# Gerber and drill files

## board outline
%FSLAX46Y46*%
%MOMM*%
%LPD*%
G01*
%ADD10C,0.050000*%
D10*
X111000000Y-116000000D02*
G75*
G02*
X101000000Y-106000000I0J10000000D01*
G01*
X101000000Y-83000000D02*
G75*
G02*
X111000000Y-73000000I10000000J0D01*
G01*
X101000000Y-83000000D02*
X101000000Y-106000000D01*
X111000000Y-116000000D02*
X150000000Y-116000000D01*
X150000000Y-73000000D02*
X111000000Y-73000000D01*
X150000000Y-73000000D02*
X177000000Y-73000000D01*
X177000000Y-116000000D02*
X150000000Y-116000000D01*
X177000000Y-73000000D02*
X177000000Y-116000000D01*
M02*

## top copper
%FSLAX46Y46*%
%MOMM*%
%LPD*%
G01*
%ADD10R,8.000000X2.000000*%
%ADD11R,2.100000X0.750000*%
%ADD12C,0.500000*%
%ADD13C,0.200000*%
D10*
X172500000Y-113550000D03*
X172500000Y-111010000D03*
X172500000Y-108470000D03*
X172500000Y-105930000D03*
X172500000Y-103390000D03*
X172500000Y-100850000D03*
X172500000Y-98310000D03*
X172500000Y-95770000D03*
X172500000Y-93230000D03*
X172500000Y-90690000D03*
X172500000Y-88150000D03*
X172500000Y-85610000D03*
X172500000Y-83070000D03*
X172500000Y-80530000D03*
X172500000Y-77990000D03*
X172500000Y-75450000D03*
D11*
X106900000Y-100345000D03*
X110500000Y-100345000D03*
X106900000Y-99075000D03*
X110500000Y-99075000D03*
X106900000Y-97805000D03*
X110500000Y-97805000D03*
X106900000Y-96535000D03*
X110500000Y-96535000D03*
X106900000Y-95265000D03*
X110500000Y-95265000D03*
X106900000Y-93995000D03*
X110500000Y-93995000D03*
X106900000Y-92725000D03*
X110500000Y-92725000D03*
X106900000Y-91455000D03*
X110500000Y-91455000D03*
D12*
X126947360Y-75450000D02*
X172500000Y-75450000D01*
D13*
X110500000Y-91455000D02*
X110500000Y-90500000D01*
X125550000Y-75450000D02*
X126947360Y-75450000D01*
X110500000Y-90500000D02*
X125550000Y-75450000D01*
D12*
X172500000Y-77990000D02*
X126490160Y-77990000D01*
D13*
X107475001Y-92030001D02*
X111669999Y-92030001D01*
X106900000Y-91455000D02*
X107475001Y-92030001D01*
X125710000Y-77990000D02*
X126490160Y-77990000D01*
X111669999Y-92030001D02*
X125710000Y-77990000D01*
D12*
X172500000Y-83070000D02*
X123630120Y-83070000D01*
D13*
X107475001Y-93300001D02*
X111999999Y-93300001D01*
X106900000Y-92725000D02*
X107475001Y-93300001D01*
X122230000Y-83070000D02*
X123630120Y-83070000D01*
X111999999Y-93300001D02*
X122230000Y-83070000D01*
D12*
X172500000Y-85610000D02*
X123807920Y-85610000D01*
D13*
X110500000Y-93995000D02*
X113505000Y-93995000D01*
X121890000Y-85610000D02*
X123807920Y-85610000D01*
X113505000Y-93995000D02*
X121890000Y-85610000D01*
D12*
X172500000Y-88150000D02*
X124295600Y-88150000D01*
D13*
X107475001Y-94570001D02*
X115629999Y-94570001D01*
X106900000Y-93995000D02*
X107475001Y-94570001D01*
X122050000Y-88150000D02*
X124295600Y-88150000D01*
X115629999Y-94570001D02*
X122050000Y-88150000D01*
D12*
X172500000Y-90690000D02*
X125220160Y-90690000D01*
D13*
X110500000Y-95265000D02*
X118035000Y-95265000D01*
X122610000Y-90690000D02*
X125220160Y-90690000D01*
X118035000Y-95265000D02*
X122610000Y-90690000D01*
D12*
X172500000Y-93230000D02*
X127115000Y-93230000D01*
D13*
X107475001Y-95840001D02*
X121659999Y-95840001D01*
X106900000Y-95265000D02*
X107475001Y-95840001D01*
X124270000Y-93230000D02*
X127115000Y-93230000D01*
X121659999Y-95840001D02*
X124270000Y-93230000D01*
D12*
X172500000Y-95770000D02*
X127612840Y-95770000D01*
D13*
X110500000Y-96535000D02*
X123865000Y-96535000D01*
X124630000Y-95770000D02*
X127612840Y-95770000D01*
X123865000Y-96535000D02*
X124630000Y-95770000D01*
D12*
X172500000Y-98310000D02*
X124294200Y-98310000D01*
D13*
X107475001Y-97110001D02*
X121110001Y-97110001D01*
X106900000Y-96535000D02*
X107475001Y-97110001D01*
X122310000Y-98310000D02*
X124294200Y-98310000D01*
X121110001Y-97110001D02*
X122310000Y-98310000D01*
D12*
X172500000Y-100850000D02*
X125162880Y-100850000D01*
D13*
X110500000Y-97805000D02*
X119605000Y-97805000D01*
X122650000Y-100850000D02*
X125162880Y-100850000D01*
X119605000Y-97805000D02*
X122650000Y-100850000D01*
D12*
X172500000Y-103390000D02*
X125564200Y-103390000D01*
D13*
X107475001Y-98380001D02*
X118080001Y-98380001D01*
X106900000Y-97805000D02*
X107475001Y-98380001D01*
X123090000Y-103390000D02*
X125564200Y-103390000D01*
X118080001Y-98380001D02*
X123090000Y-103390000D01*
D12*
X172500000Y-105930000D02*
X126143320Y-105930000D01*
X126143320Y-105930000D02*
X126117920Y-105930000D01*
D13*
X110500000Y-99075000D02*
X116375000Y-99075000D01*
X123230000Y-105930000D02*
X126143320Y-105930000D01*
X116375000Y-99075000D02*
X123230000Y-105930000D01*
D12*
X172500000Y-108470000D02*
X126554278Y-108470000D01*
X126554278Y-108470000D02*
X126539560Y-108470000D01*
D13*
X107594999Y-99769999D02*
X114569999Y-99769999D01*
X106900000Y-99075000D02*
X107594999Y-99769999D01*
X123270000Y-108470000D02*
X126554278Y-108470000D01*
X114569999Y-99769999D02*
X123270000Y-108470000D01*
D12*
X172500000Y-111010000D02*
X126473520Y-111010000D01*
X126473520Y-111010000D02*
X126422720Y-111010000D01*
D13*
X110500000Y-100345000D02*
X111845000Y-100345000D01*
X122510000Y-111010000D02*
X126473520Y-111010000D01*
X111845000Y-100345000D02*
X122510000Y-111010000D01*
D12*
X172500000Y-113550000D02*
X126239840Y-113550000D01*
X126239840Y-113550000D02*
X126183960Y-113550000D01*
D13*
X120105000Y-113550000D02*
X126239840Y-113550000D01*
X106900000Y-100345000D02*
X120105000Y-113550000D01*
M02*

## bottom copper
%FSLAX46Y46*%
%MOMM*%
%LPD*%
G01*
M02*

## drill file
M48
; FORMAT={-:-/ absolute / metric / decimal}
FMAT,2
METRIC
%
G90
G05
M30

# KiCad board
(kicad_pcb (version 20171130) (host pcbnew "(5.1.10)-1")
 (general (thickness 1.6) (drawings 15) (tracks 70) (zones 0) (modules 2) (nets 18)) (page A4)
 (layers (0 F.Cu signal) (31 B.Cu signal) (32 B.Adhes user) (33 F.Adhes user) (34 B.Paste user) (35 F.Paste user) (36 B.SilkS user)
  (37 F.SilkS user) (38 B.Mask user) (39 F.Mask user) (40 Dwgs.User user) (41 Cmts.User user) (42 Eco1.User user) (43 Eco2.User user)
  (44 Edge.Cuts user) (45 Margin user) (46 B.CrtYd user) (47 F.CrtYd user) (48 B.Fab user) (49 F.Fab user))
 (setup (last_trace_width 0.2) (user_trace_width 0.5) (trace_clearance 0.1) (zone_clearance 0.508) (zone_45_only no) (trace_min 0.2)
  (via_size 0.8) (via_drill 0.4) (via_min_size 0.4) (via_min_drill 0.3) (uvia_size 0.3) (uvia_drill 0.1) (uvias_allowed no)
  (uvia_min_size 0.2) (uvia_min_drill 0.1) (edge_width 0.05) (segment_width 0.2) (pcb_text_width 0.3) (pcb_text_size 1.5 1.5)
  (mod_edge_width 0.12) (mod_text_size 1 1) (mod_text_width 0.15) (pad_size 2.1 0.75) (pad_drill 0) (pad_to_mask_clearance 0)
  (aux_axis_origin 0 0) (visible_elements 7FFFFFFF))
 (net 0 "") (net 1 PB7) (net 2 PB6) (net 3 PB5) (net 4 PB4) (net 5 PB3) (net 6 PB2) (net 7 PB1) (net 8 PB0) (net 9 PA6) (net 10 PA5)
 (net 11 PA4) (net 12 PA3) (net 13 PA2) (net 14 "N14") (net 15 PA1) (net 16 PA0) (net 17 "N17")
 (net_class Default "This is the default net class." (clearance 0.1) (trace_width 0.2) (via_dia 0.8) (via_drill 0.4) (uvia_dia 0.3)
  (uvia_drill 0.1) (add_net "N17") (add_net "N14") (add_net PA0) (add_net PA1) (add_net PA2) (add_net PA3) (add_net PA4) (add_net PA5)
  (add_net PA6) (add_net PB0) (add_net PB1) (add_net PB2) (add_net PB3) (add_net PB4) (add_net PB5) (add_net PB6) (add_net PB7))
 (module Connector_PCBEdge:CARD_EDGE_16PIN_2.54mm (layer F.Cu) (at 172.5 94.5 90)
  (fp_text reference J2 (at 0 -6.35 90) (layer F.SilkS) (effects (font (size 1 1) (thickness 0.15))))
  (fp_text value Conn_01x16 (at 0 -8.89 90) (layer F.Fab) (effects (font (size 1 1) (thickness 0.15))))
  (pad 16 connect rect (at -19.05 0 90) (size 2 8) (layers F.Cu F.Mask) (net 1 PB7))
  (pad 15 connect rect (at -16.51 0 90) (size 2 8) (layers F.Cu F.Mask) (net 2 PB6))
  (pad 14 connect rect (at -13.97 0 90) (size 2 8) (layers F.Cu F.Mask) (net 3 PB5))
  (pad 13 connect rect (at -11.43 0 90) (size 2 8) (layers F.Cu F.Mask) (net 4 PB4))
  (pad 12 connect rect (at -8.89 0 90) (size 2 8) (layers F.Cu F.Mask) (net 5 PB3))
  (pad 11 connect rect (at -6.35 0 90) (size 2 8) (layers F.Cu F.Mask) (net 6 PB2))
  (pad 10 connect rect (at -3.81 0 90) (size 2 8) (layers F.Cu F.Mask) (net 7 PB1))
  (pad 9 connect rect (at -1.27 0 90) (size 2 8) (layers F.Cu F.Mask) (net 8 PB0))
  (pad 8 connect rect (at 1.27 0 90) (size 2 8) (layers F.Cu F.Mask) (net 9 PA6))
  (pad 7 connect rect (at 3.81 0 90) (size 2 8) (layers F.Cu F.Mask) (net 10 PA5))
  (pad 6 connect rect (at 6.35 0 90) (size 2 8) (layers F.Cu F.Mask) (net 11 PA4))
  (pad 5 connect rect (at 8.89 0 90) (size 2 8) (layers F.Cu F.Mask) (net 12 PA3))
  (pad 4 connect rect (at 11.43 0 90) (size 2 8) (layers F.Cu F.Mask) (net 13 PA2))
  (pad 3 connect rect (at 13.97 0 90) (size 2 8) (layers F.Cu F.Mask) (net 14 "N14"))
  (pad 2 connect rect (at 16.51 0 90) (size 2 8) (layers F.Cu F.Mask) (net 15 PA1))
  (pad 1 connect rect (at 19.05 0 90) (size 2 8) (layers F.Cu F.Mask) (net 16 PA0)))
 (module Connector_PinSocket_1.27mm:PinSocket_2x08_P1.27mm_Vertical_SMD (layer F.Cu) (at 108.7 95.9)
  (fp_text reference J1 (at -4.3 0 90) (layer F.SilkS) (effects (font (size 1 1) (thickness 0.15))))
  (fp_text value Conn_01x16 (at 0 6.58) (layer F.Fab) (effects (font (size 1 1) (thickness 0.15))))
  (pad 16 smd rect (at -1.8 4.445) (size 2.1 0.75) (layers F.Cu F.Paste F.Mask) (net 1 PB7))
  (pad 15 smd rect (at 1.8 4.445) (size 2.1 0.75) (layers F.Cu F.Paste F.Mask) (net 2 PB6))
  (pad 14 smd rect (at -1.8 3.175) (size 2.1 0.75) (layers F.Cu F.Paste F.Mask) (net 3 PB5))
  (pad 13 smd rect (at 1.8 3.175) (size 2.1 0.75) (layers F.Cu F.Paste F.Mask) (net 4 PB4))
  (pad 12 smd rect (at -1.8 1.905) (size 2.1 0.75) (layers F.Cu F.Paste F.Mask) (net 5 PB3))
  (pad 11 smd rect (at 1.8 1.905) (size 2.1 0.75) (layers F.Cu F.Paste F.Mask) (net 6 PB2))
  (pad 10 smd rect (at -1.8 0.635) (size 2.1 0.75) (layers F.Cu F.Paste F.Mask) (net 7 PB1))
  (pad 9 smd rect (at 1.8 0.635) (size 2.1 0.75) (layers F.Cu F.Paste F.Mask) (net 8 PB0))
  (pad 8 smd rect (at -1.8 -0.635) (size 2.1 0.75) (layers F.Cu F.Paste F.Mask) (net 9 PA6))
  (pad 7 smd rect (at 1.8 -0.635) (size 2.1 0.75) (layers F.Cu F.Paste F.Mask) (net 10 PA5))
  (pad 6 smd rect (at -1.8 -1.905) (size 2.1 0.75) (layers F.Cu F.Paste F.Mask) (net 11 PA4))
  (pad 5 smd rect (at 1.8 -1.905) (size 2.1 0.75) (layers F.Cu F.Paste F.Mask) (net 12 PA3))
  (pad 4 smd rect (at -1.8 -3.175) (size 2.1 0.75) (layers F.Cu F.Paste F.Mask) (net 13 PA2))
  (pad 3 smd rect (at 1.8 -3.175) (size 2.1 0.75) (layers F.Cu F.Paste F.Mask) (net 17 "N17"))
  (pad 2 smd rect (at -1.8 -4.445) (size 2.1 0.75) (layers F.Cu F.Paste F.Mask) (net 15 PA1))
  (pad 1 smd rect (at 1.8 -4.445) (size 2.1 0.75) (layers F.Cu F.Paste F.Mask) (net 16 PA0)))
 (gr_arc (start 111 106) (end 101 106) (angle -90) (layer Edge.Cuts) (width 0.05))
 (gr_arc (start 111 83) (end 111 73) (angle -90) (layer Edge.Cuts) (width 0.05))
 (gr_line (start 101 83) (end 101 106) (layer Edge.Cuts) (width 0.05))
 (gr_line (start 111 116) (end 150 116) (layer Edge.Cuts) (width 0.05))
 (gr_line (start 150 73) (end 111 73) (layer Edge.Cuts) (width 0.05))
 (gr_line (start 150 73) (end 177 73) (layer Edge.Cuts) (width 0.05))
 (gr_line (start 177 116) (end 150 116) (layer Edge.Cuts) (width 0.05))
 (gr_line (start 177 73) (end 177 116) (layer Edge.Cuts) (width 0.05))
 (segment (start 126.94736 75.45) (end 172.5 75.45) (width 0.5) (layer F.Cu) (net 16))
 (segment (start 110.5 91.455) (end 110.5 90.5) (width 0.2) (layer F.Cu) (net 16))
 (segment (start 125.55 75.45) (end 126.94736 75.45) (width 0.2) (layer F.Cu) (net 16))
 (segment (start 110.5 90.5) (end 125.55 75.45) (width 0.2) (layer F.Cu) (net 16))
 (segment (start 172.5 77.99) (end 126.49016 77.99) (width 0.5) (layer F.Cu) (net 15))
 (segment (start 107.475001 92.030001) (end 111.669999 92.030001) (width 0.2) (layer F.Cu) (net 15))
 (segment (start 106.9 91.455) (end 107.475001 92.030001) (width 0.2) (layer F.Cu) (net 15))
 (segment (start 125.71 77.99) (end 126.49016 77.99) (width 0.2) (layer F.Cu) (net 15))
 (segment (start 111.669999 92.030001) (end 125.71 77.99) (width 0.2) (layer F.Cu) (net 15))
 (segment (start 172.5 83.07) (end 123.63012 83.07) (width 0.5) (layer F.Cu) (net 13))
 (segment (start 107.475001 93.300001) (end 111.999999 93.300001) (width 0.2) (layer F.Cu) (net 13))
 (segment (start 106.9 92.725) (end 107.475001 93.300001) (width 0.2) (layer F.Cu) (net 13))
 (segment (start 122.23 83.07) (end 123.63012 83.07) (width 0.2) (layer F.Cu) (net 13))
 (segment (start 111.999999 93.300001) (end 122.23 83.07) (width 0.2) (layer F.Cu) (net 13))
 (segment (start 172.5 85.61) (end 123.80792 85.61) (width 0.5) (layer F.Cu) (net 12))
 (segment (start 110.5 93.995) (end 113.505 93.995) (width 0.2) (layer F.Cu) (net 12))
 (segment (start 121.89 85.61) (end 123.80792 85.61) (width 0.2) (layer F.Cu) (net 12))
 (segment (start 113.505 93.995) (end 121.89 85.61) (width 0.2) (layer F.Cu) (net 12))
 (segment (start 172.5 88.15) (end 124.2956 88.15) (width 0.5) (layer F.Cu) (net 11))
 (segment (start 107.475001 94.570001) (end 115.629999 94.570001) (width 0.2) (layer F.Cu) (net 11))
 (segment (start 106.9 93.995) (end 107.475001 94.570001) (width 0.2) (layer F.Cu) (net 11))
 (segment (start 122.05 88.15) (end 124.2956 88.15) (width 0.2) (layer F.Cu) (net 11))
 (segment (start 115.629999 94.570001) (end 122.05 88.15) (width 0.2) (layer F.Cu) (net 11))
 (segment (start 172.5 90.69) (end 125.22016 90.69) (width 0.5) (layer F.Cu) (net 10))
 (segment (start 110.5 95.265) (end 118.035 95.265) (width 0.2) (layer F.Cu) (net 10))
 (segment (start 122.61 90.69) (end 125.22016 90.69) (width 0.2) (layer F.Cu) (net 10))
 (segment (start 118.035 95.265) (end 122.61 90.69) (width 0.2) (layer F.Cu) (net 10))
 (segment (start 172.5 93.23) (end 127.115 93.23) (width 0.5) (layer F.Cu) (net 9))
 (segment (start 107.475001 95.840001) (end 121.659999 95.840001) (width 0.2) (layer F.Cu) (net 9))
 (segment (start 106.9 95.265) (end 107.475001 95.840001) (width 0.2) (layer F.Cu) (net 9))
 (segment (start 124.27 93.23) (end 127.115 93.23) (width 0.2) (layer F.Cu) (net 9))
 (segment (start 121.659999 95.840001) (end 124.27 93.23) (width 0.2) (layer F.Cu) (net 9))
 (segment (start 172.5 95.77) (end 127.61284 95.77) (width 0.5) (layer F.Cu) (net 8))
 (segment (start 110.5 96.535) (end 123.865 96.535) (width 0.2) (layer F.Cu) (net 8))
 (segment (start 124.63 95.77) (end 127.61284 95.77) (width 0.2) (layer F.Cu) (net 8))
 (segment (start 123.865 96.535) (end 124.63 95.77) (width 0.2) (layer F.Cu) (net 8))
 (segment (start 172.5 98.31) (end 124.2942 98.31) (width 0.5) (layer F.Cu) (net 7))
 (segment (start 107.475001 97.110001) (end 121.110001 97.110001) (width 0.2) (layer F.Cu) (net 7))
 (segment (start 106.9 96.535) (end 107.475001 97.110001) (width 0.2) (layer F.Cu) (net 7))
 (segment (start 122.31 98.31) (end 124.2942 98.31) (width 0.2) (layer F.Cu) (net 7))
 (segment (start 121.110001 97.110001) (end 122.31 98.31) (width 0.2) (layer F.Cu) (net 7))
 (segment (start 172.5 100.85) (end 125.16288 100.85) (width 0.5) (layer F.Cu) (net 6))
 (segment (start 110.5 97.805) (end 119.605 97.805) (width 0.2) (layer F.Cu) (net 6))
 (segment (start 122.65 100.85) (end 125.16288 100.85) (width 0.2) (layer F.Cu) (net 6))
 (segment (start 119.605 97.805) (end 122.65 100.85) (width 0.2) (layer F.Cu) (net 6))
 (segment (start 172.5 103.39) (end 125.5642 103.39) (width 0.5) (layer F.Cu) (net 5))
 (segment (start 107.475001 98.380001) (end 118.080001 98.380001) (width 0.2) (layer F.Cu) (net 5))
 (segment (start 106.9 97.805) (end 107.475001 98.380001) (width 0.2) (layer F.Cu) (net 5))
 (segment (start 123.09 103.39) (end 125.5642 103.39) (width 0.2) (layer F.Cu) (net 5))
 (segment (start 118.080001 98.380001) (end 123.09 103.39) (width 0.2) (layer F.Cu) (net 5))
 (segment (start 172.5 105.93) (end 126.14332 105.93) (width 0.5) (layer F.Cu) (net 4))
 (segment (start 126.14332 105.93) (end 126.11792 105.93) (width 0.5) (layer F.Cu) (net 4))
 (segment (start 110.5 99.075) (end 116.375 99.075) (width 0.2) (layer F.Cu) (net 4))
 (segment (start 123.23 105.93) (end 126.14332 105.93) (width 0.2) (layer F.Cu) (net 4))
 (segment (start 116.375 99.075) (end 123.23 105.93) (width 0.2) (layer F.Cu) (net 4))
 (segment (start 172.5 108.47) (end 126.554278 108.47) (width 0.5) (layer F.Cu) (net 3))
 (segment (start 126.554278 108.47) (end 126.53956 108.47) (width 0.5) (layer F.Cu) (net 3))
 (segment (start 107.594999 99.769999) (end 114.569999 99.769999) (width 0.2) (layer F.Cu) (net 3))
 (segment (start 106.9 99.075) (end 107.594999 99.769999) (width 0.2) (layer F.Cu) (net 3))
 (segment (start 123.27 108.47) (end 126.554278 108.47) (width 0.2) (layer F.Cu) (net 3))
 (segment (start 114.569999 99.769999) (end 123.27 108.47) (width 0.2) (layer F.Cu) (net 3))
 (segment (start 172.5 111.01) (end 126.47352 111.01) (width 0.5) (layer F.Cu) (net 2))
 (segment (start 126.47352 111.01) (end 126.42272 111.01) (width 0.5) (layer F.Cu) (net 2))
 (segment (start 110.5 100.345) (end 111.845 100.345) (width 0.2) (layer F.Cu) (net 2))
 (segment (start 122.51 111.01) (end 126.47352 111.01) (width 0.2) (layer F.Cu) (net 2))
 (segment (start 111.845 100.345) (end 122.51 111.01) (width 0.2) (layer F.Cu) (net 2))
 (segment (start 172.5 113.55) (end 126.23984 113.55) (width 0.5) (layer F.Cu) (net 1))
 (segment (start 126.23984 113.55) (end 126.18396 113.55) (width 0.5) (layer F.Cu) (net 1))
 (segment (start 120.105 113.55) (end 126.23984 113.55) (width 0.2) (layer F.Cu) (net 1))
 (segment (start 106.9 100.345) (end 120.105 113.55) (width 0.2) (layer F.Cu) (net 1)))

